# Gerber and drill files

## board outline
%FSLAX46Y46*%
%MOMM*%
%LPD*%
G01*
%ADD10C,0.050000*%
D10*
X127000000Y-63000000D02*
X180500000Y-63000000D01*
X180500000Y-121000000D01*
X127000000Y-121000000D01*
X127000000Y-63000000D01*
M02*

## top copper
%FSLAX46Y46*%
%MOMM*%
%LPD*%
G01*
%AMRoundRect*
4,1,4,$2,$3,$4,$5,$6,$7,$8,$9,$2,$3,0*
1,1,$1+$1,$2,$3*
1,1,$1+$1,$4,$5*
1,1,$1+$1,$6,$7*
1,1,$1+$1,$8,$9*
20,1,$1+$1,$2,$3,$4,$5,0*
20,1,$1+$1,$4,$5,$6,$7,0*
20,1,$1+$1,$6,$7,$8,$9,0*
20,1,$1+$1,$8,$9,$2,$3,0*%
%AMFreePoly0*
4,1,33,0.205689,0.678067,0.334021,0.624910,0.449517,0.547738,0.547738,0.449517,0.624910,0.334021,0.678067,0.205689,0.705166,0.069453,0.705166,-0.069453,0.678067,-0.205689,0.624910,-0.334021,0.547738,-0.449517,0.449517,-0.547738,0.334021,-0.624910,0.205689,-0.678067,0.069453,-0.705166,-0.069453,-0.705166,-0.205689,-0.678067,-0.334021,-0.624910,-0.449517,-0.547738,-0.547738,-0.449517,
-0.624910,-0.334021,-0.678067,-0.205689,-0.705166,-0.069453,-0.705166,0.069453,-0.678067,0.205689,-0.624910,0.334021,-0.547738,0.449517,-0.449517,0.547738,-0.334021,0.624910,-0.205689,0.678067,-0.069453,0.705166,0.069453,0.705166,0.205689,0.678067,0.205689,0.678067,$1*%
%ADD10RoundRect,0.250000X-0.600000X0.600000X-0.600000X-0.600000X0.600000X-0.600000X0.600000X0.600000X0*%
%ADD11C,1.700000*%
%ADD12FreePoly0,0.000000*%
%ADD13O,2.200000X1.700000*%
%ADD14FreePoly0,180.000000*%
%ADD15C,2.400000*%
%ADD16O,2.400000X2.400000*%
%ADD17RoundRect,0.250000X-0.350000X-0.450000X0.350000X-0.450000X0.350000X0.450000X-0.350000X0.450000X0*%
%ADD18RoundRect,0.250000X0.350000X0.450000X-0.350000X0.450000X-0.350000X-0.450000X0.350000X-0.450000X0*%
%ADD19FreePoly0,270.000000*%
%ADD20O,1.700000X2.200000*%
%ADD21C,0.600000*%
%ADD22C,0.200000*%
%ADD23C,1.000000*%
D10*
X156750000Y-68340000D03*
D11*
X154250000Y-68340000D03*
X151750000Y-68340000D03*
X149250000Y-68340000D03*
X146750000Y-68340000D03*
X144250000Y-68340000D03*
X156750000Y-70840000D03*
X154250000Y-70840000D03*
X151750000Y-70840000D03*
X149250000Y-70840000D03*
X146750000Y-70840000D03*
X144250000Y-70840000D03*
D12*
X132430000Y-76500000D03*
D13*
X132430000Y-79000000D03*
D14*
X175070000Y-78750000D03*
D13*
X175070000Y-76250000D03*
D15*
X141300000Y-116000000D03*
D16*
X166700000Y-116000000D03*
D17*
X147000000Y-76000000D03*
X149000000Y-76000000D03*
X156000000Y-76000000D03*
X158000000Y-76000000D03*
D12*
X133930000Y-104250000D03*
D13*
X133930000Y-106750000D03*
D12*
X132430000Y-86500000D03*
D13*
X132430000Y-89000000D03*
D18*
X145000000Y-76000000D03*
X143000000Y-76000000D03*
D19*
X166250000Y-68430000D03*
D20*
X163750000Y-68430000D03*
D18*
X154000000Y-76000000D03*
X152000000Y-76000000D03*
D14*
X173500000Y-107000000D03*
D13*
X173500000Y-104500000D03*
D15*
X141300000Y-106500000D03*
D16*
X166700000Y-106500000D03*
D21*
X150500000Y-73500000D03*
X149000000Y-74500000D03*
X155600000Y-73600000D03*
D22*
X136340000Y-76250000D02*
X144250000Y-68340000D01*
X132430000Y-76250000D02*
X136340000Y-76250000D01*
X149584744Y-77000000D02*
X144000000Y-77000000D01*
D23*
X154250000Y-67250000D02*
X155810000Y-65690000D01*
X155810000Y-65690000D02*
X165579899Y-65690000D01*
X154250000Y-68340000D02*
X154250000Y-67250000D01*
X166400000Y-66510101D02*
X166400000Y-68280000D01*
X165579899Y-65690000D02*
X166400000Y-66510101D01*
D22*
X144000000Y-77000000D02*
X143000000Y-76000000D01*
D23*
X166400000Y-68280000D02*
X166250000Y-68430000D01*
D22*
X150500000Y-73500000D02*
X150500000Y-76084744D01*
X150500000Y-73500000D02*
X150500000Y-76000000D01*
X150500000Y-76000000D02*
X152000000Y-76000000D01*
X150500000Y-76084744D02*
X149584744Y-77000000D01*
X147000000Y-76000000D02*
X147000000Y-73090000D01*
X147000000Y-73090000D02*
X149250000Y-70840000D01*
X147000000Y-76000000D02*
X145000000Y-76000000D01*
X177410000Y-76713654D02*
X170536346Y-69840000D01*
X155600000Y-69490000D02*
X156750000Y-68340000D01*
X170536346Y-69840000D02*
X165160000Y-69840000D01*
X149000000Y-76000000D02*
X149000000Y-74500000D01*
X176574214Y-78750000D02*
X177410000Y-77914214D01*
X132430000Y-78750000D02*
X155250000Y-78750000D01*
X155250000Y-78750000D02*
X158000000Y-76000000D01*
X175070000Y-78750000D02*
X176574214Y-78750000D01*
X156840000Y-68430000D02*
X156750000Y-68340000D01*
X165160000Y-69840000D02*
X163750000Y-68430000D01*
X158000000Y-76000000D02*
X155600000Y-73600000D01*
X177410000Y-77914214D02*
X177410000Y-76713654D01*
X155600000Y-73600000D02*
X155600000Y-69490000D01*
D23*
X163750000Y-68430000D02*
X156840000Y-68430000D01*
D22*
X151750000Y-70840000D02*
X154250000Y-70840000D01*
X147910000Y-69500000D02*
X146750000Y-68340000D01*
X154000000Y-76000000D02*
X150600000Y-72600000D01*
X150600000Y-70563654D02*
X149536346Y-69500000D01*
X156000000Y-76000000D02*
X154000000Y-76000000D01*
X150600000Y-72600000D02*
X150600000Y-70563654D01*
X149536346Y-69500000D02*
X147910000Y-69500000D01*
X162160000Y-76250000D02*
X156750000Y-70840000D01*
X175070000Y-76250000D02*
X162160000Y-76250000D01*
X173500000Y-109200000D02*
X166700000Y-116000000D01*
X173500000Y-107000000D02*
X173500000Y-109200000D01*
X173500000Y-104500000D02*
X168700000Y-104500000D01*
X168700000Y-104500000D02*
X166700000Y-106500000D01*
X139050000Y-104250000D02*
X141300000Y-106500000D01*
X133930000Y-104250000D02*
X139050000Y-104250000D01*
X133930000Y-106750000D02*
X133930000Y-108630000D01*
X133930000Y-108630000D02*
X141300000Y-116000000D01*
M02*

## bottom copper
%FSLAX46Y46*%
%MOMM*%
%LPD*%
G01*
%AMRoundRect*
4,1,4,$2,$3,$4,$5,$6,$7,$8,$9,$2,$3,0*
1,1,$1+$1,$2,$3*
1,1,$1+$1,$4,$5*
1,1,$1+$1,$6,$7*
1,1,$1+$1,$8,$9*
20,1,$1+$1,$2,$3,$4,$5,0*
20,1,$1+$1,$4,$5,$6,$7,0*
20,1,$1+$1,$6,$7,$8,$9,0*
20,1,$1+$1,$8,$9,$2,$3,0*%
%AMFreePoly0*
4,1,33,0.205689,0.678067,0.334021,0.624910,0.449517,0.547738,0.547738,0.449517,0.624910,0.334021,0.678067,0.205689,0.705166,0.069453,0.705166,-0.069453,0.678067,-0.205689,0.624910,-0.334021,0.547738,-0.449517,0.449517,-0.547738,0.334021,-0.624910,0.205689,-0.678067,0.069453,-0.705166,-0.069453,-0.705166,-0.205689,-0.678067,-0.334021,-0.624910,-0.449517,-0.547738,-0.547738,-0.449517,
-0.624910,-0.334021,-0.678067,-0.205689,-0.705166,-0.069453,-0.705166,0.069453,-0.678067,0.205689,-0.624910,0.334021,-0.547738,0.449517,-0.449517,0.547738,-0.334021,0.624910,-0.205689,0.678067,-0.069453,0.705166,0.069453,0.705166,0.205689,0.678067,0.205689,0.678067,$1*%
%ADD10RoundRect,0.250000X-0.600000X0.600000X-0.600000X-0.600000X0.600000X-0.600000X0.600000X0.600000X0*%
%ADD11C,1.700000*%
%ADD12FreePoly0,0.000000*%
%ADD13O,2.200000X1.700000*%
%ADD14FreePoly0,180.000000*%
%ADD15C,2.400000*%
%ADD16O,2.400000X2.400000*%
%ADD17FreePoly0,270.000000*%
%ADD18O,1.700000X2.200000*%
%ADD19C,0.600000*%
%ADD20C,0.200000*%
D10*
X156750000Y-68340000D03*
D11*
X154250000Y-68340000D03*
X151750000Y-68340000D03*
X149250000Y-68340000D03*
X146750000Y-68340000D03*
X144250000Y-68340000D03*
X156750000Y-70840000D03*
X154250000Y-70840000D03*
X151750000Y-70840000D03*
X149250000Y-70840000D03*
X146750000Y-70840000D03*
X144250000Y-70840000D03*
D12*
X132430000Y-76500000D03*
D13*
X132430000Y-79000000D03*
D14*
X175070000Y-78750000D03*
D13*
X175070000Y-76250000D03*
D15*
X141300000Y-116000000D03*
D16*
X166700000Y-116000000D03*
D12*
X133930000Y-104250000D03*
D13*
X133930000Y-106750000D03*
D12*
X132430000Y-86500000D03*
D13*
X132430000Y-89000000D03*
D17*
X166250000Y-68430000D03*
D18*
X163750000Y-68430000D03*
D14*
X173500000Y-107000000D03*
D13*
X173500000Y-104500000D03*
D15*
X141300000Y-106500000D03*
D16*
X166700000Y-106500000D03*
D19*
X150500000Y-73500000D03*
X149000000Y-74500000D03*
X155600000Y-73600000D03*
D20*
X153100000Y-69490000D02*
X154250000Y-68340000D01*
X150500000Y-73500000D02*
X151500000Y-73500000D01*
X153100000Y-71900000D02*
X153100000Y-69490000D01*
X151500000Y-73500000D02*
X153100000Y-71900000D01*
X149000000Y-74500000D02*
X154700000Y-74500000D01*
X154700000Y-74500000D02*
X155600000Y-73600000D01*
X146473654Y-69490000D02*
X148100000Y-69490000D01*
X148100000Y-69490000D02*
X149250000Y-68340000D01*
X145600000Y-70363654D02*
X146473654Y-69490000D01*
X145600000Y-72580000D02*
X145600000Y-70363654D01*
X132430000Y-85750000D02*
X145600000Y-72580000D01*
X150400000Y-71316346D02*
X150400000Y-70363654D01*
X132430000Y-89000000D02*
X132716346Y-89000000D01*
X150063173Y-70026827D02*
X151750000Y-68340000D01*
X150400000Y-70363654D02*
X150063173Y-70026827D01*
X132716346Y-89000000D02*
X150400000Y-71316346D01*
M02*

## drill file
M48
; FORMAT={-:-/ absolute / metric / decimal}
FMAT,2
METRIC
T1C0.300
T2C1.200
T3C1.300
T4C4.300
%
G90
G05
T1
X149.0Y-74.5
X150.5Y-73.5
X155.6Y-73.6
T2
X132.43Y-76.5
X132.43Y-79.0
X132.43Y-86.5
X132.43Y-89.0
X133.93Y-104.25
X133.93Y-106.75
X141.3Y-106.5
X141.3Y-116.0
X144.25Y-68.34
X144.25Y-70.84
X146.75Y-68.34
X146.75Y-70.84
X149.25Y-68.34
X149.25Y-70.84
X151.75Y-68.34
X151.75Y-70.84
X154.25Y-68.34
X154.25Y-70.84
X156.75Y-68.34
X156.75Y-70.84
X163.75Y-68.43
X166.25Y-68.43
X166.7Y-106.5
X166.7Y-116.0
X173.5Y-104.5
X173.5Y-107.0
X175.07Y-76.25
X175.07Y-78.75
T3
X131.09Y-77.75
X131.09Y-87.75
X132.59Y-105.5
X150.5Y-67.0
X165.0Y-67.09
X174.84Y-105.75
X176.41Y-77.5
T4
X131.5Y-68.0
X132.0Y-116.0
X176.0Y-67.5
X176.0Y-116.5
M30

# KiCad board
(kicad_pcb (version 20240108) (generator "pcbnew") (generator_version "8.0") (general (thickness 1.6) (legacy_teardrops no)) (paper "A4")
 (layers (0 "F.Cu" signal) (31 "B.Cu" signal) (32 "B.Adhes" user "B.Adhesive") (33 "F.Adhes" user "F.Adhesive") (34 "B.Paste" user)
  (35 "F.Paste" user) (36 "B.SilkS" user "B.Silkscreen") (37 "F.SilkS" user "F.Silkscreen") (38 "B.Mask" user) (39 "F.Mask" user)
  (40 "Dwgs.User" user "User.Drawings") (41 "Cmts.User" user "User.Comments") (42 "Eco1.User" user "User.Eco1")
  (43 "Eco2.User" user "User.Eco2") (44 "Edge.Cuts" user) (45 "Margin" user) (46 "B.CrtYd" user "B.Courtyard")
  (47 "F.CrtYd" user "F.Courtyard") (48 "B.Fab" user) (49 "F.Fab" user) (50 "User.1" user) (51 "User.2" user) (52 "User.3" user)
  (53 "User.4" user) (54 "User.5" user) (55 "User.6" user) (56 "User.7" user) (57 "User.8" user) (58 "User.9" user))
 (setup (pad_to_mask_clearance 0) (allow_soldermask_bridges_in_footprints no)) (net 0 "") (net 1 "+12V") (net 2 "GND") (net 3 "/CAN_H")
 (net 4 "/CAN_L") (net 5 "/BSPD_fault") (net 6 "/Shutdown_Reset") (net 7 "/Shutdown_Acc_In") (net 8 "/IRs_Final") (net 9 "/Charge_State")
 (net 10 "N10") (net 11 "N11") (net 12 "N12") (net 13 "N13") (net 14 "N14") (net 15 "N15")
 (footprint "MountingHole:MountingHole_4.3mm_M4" (layer "F.Cu") (at 176 116.5)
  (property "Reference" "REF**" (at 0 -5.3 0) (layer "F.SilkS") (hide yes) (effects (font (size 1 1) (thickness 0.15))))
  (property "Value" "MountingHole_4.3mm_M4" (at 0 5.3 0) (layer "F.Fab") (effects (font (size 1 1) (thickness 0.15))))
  (pad "" np_thru_hole circle (at 0 0) (size 4.3 4.3) (drill 4.3) (layers "*.Cu" "*.Mask")))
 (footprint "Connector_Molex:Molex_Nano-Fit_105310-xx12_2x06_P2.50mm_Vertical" (layer "F.Cu") (at 156.75 68.34 -90)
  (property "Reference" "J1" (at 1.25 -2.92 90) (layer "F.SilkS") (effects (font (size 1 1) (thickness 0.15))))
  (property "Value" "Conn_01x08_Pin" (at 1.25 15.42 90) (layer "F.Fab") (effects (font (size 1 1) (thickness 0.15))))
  (pad "" np_thru_hole circle (at -1.34 6.25 270) (size 1.3 1.3) (drill 1.3) (layers "*.Cu" "*.Mask"))
  (pad "1" thru_hole roundrect (at 0 0 270) (size 1.7 1.7) (drill 1.2) (layers "*.Cu" "*.Mask") (remove_unused_layers no)
   (roundrect_rratio 0.147059) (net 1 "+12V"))
  (pad "2" thru_hole circle (at 0 2.5 270) (size 1.7 1.7) (drill 1.2) (layers "*.Cu" "*.Mask") (remove_unused_layers no) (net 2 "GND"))
  (pad "3" thru_hole circle (at 0 5 270) (size 1.7 1.7) (drill 1.2) (layers "*.Cu" "*.Mask") (remove_unused_layers no) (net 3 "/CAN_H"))
  (pad "4" thru_hole circle (at 0 7.5 270) (size 1.7 1.7) (drill 1.2) (layers "*.Cu" "*.Mask") (remove_unused_layers no) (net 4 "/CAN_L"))
  (pad "5" thru_hole circle (at 0 10 270) (size 1.7 1.7) (drill 1.2) (layers "*.Cu" "*.Mask") (remove_unused_layers no)
   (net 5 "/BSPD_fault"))
  (pad "6" thru_hole circle (at 0 12.5 270) (size 1.7 1.7) (drill 1.2) (layers "*.Cu" "*.Mask") (remove_unused_layers no)
   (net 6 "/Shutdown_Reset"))
  (pad "7" thru_hole circle (at 2.5 0 270) (size 1.7 1.7) (drill 1.2) (layers "*.Cu" "*.Mask") (remove_unused_layers no)
   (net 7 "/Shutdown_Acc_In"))
  (pad "8" thru_hole circle (at 2.5 2.5 270) (size 1.7 1.7) (drill 1.2) (layers "*.Cu" "*.Mask") (remove_unused_layers no)
   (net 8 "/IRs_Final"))
  (pad "9" thru_hole circle (at 2.5 5 270) (size 1.7 1.7) (drill 1.2) (layers "*.Cu" "*.Mask") (remove_unused_layers no)
   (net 8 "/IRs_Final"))
  (pad "10" thru_hole circle (at 2.5 7.5 270) (size 1.7 1.7) (drill 1.2) (layers "*.Cu" "*.Mask") (remove_unused_layers no)
   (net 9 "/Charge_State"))
  (pad "11" thru_hole circle (at 2.5 10 270) (size 1.7 1.7) (drill 1.2) (layers "*.Cu" "*.Mask") (remove_unused_layers no) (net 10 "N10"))
  (pad "12" thru_hole circle (at 2.5 12.5 270) (size 1.7 1.7) (drill 1.2) (layers "*.Cu" "*.Mask") (remove_unused_layers no) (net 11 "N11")))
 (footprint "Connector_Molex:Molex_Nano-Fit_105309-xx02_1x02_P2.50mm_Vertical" (layer "F.Cu") (at 132.43 76.5)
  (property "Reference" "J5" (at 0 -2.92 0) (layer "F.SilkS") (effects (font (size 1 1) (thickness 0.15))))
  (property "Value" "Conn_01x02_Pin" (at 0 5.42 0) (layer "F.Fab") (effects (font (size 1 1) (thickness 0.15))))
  (pad "" np_thru_hole circle (at -1.34 1.25) (size 1.3 1.3) (drill 1.3) (layers "*.Cu" "*.Mask"))
  (pad "1" thru_hole custom (at 0 0) (size 1.417157 1.417157) (drill 1.2) (layers "*.Cu" "*.Mask") (remove_unused_layers no)
   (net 6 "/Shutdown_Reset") (thermal_bridge_angle 90) (options (clearance outline) (anchor circle)) (primitives))
  (pad "2" thru_hole oval (at 0 2.5) (size 2.2 1.7) (drill 1.2) (layers "*.Cu" "*.Mask") (remove_unused_layers no) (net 1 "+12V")))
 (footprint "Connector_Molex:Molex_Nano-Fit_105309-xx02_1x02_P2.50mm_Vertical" (layer "F.Cu") (at 175.07 78.75 180)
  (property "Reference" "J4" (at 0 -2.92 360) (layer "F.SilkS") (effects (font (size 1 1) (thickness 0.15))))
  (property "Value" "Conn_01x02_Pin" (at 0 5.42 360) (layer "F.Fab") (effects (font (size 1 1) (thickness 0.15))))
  (pad "" np_thru_hole circle (at -1.34 1.25 180) (size 1.3 1.3) (drill 1.3) (layers "*.Cu" "*.Mask"))
  (pad "1" thru_hole custom (at 0 0 180) (size 1.417157 1.417157) (drill 1.2) (layers "*.Cu" "*.Mask") (remove_unused_layers no)
   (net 1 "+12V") (thermal_bridge_angle 90) (options (clearance outline) (anchor circle)) (primitives))
  (pad "2" thru_hole oval (at 0 2.5 180) (size 2.2 1.7) (drill 1.2) (layers "*.Cu" "*.Mask") (remove_unused_layers no)
   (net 7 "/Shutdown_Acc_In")))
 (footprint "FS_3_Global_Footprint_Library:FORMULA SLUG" (layer "F.Cu") (at 146 87.975292)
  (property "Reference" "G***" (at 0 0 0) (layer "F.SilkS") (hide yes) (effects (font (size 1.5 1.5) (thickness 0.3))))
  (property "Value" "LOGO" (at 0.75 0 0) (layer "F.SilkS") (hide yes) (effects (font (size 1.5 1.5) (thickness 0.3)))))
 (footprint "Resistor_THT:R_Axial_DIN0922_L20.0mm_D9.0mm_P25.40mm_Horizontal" (layer "F.Cu") (at 141.3 116)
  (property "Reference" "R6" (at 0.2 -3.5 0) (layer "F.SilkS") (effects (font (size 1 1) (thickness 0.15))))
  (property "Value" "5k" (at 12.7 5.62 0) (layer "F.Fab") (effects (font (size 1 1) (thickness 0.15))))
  (pad "1" thru_hole circle (at 0 0) (size 2.4 2.4) (drill 1.2) (layers "*.Cu" "*.Mask") (remove_unused_layers no) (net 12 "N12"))
  (pad "2" thru_hole oval (at 25.4 0) (size 2.4 2.4) (drill 1.2) (layers "*.Cu" "*.Mask") (remove_unused_layers no) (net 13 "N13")))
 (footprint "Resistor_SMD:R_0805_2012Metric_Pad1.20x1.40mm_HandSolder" (layer "F.Cu") (at 148 76)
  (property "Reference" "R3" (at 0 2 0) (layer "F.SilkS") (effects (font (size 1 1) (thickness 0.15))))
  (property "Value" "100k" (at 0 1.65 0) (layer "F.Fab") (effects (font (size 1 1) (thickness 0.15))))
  (pad "1" smd roundrect (at -1 0) (size 1.2 1.4) (layers "F.Cu" "F.Paste" "F.Mask") (roundrect_rratio 0.208333) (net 9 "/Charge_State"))
  (pad "2" smd roundrect (at 1 0) (size 1.2 1.4) (layers "F.Cu" "F.Paste" "F.Mask") (roundrect_rratio 0.208333) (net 1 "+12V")))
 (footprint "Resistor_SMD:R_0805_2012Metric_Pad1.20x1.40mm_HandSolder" (layer "F.Cu") (at 157 76)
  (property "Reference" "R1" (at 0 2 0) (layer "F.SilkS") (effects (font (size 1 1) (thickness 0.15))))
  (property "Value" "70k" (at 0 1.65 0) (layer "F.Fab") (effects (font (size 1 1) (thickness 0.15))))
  (pad "1" smd roundrect (at -1 0) (size 1.2 1.4) (layers "F.Cu" "F.Paste" "F.Mask") (roundrect_rratio 0.208333) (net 5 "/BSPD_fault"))
  (pad "2" smd roundrect (at 1 0) (size 1.2 1.4) (layers "F.Cu" "F.Paste" "F.Mask") (roundrect_rratio 0.208333) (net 1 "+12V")))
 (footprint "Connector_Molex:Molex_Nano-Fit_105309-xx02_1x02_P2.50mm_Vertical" (layer "F.Cu") (at 133.93 104.25)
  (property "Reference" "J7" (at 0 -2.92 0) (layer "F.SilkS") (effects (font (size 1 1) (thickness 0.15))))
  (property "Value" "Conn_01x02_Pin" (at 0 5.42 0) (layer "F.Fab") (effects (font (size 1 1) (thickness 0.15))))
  (pad "" np_thru_hole circle (at -1.34 1.25) (size 1.3 1.3) (drill 1.3) (layers "*.Cu" "*.Mask"))
  (pad "1" thru_hole custom (at 0 0) (size 1.417157 1.417157) (drill 1.2) (layers "*.Cu" "*.Mask") (remove_unused_layers no) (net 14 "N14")
   (thermal_bridge_angle 90) (options (clearance outline) (anchor circle)) (primitives))
  (pad "2" thru_hole oval (at 0 2.5) (size 2.2 1.7) (drill 1.2) (layers "*.Cu" "*.Mask") (remove_unused_layers no) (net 12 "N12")))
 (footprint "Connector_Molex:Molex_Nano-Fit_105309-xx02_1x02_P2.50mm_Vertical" (layer "F.Cu") (at 132.43 86.5)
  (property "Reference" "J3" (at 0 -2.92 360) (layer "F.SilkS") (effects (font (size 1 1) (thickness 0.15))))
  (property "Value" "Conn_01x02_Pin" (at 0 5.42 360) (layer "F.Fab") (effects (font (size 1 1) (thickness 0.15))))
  (pad "" np_thru_hole circle (at -1.34 1.25) (size 1.3 1.3) (drill 1.3) (layers "*.Cu" "*.Mask"))
  (pad "1" thru_hole custom (at 0 0) (size 1.417157 1.417157) (drill 1.2) (layers "*.Cu" "*.Mask") (remove_unused_layers no)
   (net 4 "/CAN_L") (thermal_bridge_angle 90) (options (clearance outline) (anchor circle)) (primitives))
  (pad "2" thru_hole oval (at 0 2.5) (size 2.2 1.7) (drill 1.2) (layers "*.Cu" "*.Mask") (remove_unused_layers no) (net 3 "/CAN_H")))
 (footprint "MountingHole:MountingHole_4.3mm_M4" (layer "F.Cu") (at 132 116)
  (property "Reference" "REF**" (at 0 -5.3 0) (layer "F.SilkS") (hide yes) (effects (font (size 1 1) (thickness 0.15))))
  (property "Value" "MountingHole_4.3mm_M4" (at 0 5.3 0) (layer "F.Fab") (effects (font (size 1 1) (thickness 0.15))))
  (pad "" np_thru_hole circle (at 0 0) (size 4.3 4.3) (drill 4.3) (layers "*.Cu" "*.Mask")))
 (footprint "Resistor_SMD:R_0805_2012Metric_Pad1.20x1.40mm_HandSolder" (layer "F.Cu") (at 144 76 180)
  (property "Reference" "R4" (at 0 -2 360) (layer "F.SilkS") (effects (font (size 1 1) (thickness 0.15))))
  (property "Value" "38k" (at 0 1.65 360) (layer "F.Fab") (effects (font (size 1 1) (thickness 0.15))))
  (pad "1" smd roundrect (at -1 0 180) (size 1.2 1.4) (layers "F.Cu" "F.Paste" "F.Mask") (roundrect_rratio 0.208333) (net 9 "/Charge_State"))
  (pad "2" smd roundrect (at 1 0 180) (size 1.2 1.4) (layers "F.Cu" "F.Paste" "F.Mask") (roundrect_rratio 0.208333) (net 2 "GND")))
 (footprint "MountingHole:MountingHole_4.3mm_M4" (layer "F.Cu") (at 131.5 68)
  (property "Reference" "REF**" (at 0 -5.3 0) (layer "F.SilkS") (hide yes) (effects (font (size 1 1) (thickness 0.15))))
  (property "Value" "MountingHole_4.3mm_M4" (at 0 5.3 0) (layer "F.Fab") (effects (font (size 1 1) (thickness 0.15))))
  (pad "" np_thru_hole circle (at 0 0) (size 4.3 4.3) (drill 4.3) (layers "*.Cu" "*.Mask")))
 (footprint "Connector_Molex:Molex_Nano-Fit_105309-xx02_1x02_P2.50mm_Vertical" (layer "F.Cu") (at 166.25 68.43 -90)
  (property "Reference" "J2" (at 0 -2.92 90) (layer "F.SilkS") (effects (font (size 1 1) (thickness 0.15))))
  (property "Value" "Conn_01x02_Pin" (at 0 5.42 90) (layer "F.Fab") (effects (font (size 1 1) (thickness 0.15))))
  (pad "" np_thru_hole circle (at -1.34 1.25 270) (size 1.3 1.3) (drill 1.3) (layers "*.Cu" "*.Mask"))
  (pad "1" thru_hole custom (at 0 0 270) (size 1.417157 1.417157) (drill 1.2) (layers "*.Cu" "*.Mask") (remove_unused_layers no)
   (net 2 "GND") (thermal_bridge_angle 90) (options (clearance outline) (anchor circle)) (primitives))
  (pad "2" thru_hole oval (at 0 2.5 270) (size 2.2 1.7) (drill 1.2) (layers "*.Cu" "*.Mask") (remove_unused_layers no) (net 1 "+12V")))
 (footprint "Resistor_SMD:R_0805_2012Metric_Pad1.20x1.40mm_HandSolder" (layer "F.Cu") (at 153 76 180)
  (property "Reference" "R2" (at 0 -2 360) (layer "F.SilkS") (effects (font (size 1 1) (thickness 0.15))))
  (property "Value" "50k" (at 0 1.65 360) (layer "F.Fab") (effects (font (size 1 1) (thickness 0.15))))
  (pad "1" smd roundrect (at -1 0 180) (size 1.2 1.4) (layers "F.Cu" "F.Paste" "F.Mask") (roundrect_rratio 0.208333) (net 5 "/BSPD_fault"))
  (pad "2" smd roundrect (at 1 0 180) (size 1.2 1.4) (layers "F.Cu" "F.Paste" "F.Mask") (roundrect_rratio 0.208333) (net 2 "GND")))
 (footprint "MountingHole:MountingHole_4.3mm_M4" (layer "F.Cu") (at 176 67.5)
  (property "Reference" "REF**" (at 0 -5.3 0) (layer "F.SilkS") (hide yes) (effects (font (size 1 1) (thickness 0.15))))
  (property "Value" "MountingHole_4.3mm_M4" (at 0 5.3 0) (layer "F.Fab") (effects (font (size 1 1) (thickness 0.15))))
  (pad "" np_thru_hole circle (at 0 0) (size 4.3 4.3) (drill 4.3) (layers "*.Cu" "*.Mask")))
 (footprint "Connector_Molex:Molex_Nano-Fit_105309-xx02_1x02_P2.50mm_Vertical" (layer "F.Cu") (at 173.5 107 180)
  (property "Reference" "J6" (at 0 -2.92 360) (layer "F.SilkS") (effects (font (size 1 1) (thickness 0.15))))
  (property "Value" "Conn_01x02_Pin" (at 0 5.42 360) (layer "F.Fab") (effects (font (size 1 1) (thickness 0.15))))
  (pad "" np_thru_hole circle (at -1.34 1.25 180) (size 1.3 1.3) (drill 1.3) (layers "*.Cu" "*.Mask"))
  (pad "1" thru_hole custom (at 0 0 180) (size 1.417157 1.417157) (drill 1.2) (layers "*.Cu" "*.Mask") (remove_unused_layers no)
   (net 13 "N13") (thermal_bridge_angle 90) (options (clearance outline) (anchor circle)) (primitives))
  (pad "2" thru_hole oval (at 0 2.5 180) (size 2.2 1.7) (drill 1.2) (layers "*.Cu" "*.Mask") (remove_unused_layers no) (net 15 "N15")))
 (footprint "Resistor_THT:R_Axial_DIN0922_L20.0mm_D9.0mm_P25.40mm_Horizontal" (layer "F.Cu") (at 141.3 106.5)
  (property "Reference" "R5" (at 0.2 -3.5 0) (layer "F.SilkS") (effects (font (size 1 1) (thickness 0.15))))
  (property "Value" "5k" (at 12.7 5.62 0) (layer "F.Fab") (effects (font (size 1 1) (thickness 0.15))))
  (pad "1" thru_hole circle (at 0 0) (size 2.4 2.4) (drill 1.2) (layers "*.Cu" "*.Mask") (remove_unused_layers no) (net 14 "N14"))
  (pad "2" thru_hole oval (at 25.4 0) (size 2.4 2.4) (drill 1.2) (layers "*.Cu" "*.Mask") (remove_unused_layers no) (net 15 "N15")))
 (gr_rect (start 127 63) (end 180.5 121) (stroke (width 0.05) (type default)) (fill none) (layer "Edge.Cuts"))
 (segment (start 136.34 76.25) (end 144.25 68.34) (width 0.2) (layer "F.Cu") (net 6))
 (segment (start 132.43 76.25) (end 136.34 76.25) (width 0.2) (layer "F.Cu") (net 6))
 (segment (start 149.584744 77) (end 144 77) (width 0.2) (layer "F.Cu") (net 2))
 (segment (start 154.25 67.25) (end 155.81 65.69) (width 1) (layer "F.Cu") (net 2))
 (segment (start 155.81 65.69) (end 165.579899 65.69) (width 1) (layer "F.Cu") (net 2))
 (segment (start 154.25 68.34) (end 154.25 67.25) (width 1) (layer "F.Cu") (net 2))
 (segment (start 166.4 66.510101) (end 166.4 68.28) (width 1) (layer "F.Cu") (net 2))
 (segment (start 165.579899 65.69) (end 166.4 66.510101) (width 1) (layer "F.Cu") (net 2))
 (segment (start 144 77) (end 143 76) (width 0.2) (layer "F.Cu") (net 2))
 (segment (start 166.4 68.28) (end 166.25 68.43) (width 1) (layer "F.Cu") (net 2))
 (segment (start 150.5 73.5) (end 150.5 76.084744) (width 0.2) (layer "F.Cu") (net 2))
 (segment (start 150.5 73.5) (end 150.5 76) (width 0.2) (layer "F.Cu") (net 2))
 (segment (start 150.5 76) (end 152 76) (width 0.2) (layer "F.Cu") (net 2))
 (segment (start 150.5 76.084744) (end 149.584744 77) (width 0.2) (layer "F.Cu") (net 2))
 (via (at 150.5 73.5) (size 0.6) (drill 0.3) (layers "F.Cu" "B.Cu") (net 2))
 (segment (start 153.1 69.49) (end 154.25 68.34) (width 0.2) (layer "B.Cu") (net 2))
 (segment (start 150.5 73.5) (end 151.5 73.5) (width 0.2) (layer "B.Cu") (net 2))
 (segment (start 153.1 71.9) (end 153.1 69.49) (width 0.2) (layer "B.Cu") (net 2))
 (segment (start 151.5 73.5) (end 153.1 71.9) (width 0.2) (layer "B.Cu") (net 2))
 (segment (start 147 76) (end 147 73.09) (width 0.2) (layer "F.Cu") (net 9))
 (segment (start 147 73.09) (end 149.25 70.84) (width 0.2) (layer "F.Cu") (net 9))
 (segment (start 147 76) (end 145 76) (width 0.2) (layer "F.Cu") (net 9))
 (segment (start 177.41 76.713654) (end 170.536346 69.84) (width 0.2) (layer "F.Cu") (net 1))
 (segment (start 155.6 69.49) (end 156.75 68.34) (width 0.2) (layer "F.Cu") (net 1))
 (segment (start 170.536346 69.84) (end 165.16 69.84) (width 0.2) (layer "F.Cu") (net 1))
 (segment (start 149 76) (end 149 74.5) (width 0.2) (layer "F.Cu") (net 1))
 (segment (start 176.574214 78.75) (end 177.41 77.914214) (width 0.2) (layer "F.Cu") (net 1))
 (segment (start 132.43 78.75) (end 155.25 78.75) (width 0.2) (layer "F.Cu") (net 1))
 (segment (start 155.25 78.75) (end 158 76) (width 0.2) (layer "F.Cu") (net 1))
 (segment (start 175.07 78.75) (end 176.574214 78.75) (width 0.2) (layer "F.Cu") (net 1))
 (segment (start 156.84 68.43) (end 156.75 68.34) (width 0.2) (layer "F.Cu") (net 1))
 (segment (start 165.16 69.84) (end 163.75 68.43) (width 0.2) (layer "F.Cu") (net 1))
 (segment (start 158 76) (end 155.6 73.6) (width 0.2) (layer "F.Cu") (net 1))
 (segment (start 177.41 77.914214) (end 177.41 76.713654) (width 0.2) (layer "F.Cu") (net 1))
 (segment (start 155.6 73.6) (end 155.6 69.49) (width 0.2) (layer "F.Cu") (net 1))
 (segment (start 163.75 68.43) (end 156.84 68.43) (width 1) (layer "F.Cu") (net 1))
 (via (at 149 74.5) (size 0.6) (drill 0.3) (layers "F.Cu" "B.Cu") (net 1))
 (via (at 155.6 73.6) (size 0.6) (drill 0.3) (layers "F.Cu" "B.Cu") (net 1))
 (segment (start 149 74.5) (end 154.7 74.5) (width 0.2) (layer "B.Cu") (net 1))
 (segment (start 154.7 74.5) (end 155.6 73.6) (width 0.2) (layer "B.Cu") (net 1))
 (segment (start 151.75 70.84) (end 154.25 70.84) (width 0.2) (layer "F.Cu") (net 8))
 (segment (start 147.91 69.5) (end 146.75 68.34) (width 0.2) (layer "F.Cu") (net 5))
 (segment (start 154 76) (end 150.6 72.6) (width 0.2) (layer "F.Cu") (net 5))
 (segment (start 150.6 70.563654) (end 149.536346 69.5) (width 0.2) (layer "F.Cu") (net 5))
 (segment (start 156 76) (end 154 76) (width 0.2) (layer "F.Cu") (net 5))
 (segment (start 150.6 72.6) (end 150.6 70.563654) (width 0.2) (layer "F.Cu") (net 5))
 (segment (start 149.536346 69.5) (end 147.91 69.5) (width 0.2) (layer "F.Cu") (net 5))
 (segment (start 146.473654 69.49) (end 148.1 69.49) (width 0.2) (layer "B.Cu") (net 4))
 (segment (start 148.1 69.49) (end 149.25 68.34) (width 0.2) (layer "B.Cu") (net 4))
 (segment (start 145.6 70.363654) (end 146.473654 69.49) (width 0.2) (layer "B.Cu") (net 4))
 (segment (start 145.6 72.58) (end 145.6 70.363654) (width 0.2) (layer "B.Cu") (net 4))
 (segment (start 132.43 85.75) (end 145.6 72.58) (width 0.2) (layer "B.Cu") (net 4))
 (segment (start 162.16 76.25) (end 156.75 70.84) (width 0.2) (layer "F.Cu") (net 7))
 (segment (start 175.07 76.25) (end 162.16 76.25) (width 0.2) (layer "F.Cu") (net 7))
 (segment (start 150.4 71.316346) (end 150.4 70.363654) (width 0.2) (layer "B.Cu") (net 3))
 (segment (start 132.43 89) (end 132.716346 89) (width 0.2) (layer "B.Cu") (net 3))
 (segment (start 150.063173 70.026827) (end 151.75 68.34) (width 0.2) (layer "B.Cu") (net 3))
 (segment (start 150.4 70.363654) (end 150.063173 70.026827) (width 0.2) (layer "B.Cu") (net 3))
 (segment (start 132.716346 89) (end 150.4 71.316346) (width 0.2) (layer "B.Cu") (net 3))
 (segment (start 173.5 109.2) (end 166.7 116) (width 0.2) (layer "F.Cu") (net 13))
 (segment (start 173.5 107) (end 173.5 109.2) (width 0.2) (layer "F.Cu") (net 13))
 (segment (start 173.5 104.5) (end 168.7 104.5) (width 0.2) (layer "F.Cu") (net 15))
 (segment (start 168.7 104.5) (end 166.7 106.5) (width 0.2) (layer "F.Cu") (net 15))
 (segment (start 139.05 104.25) (end 141.3 106.5) (width 0.2) (layer "F.Cu") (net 14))
 (segment (start 133.93 104.25) (end 139.05 104.25) (width 0.2) (layer "F.Cu") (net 14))
 (segment (start 133.93 106.75) (end 133.93 108.63) (width 0.2) (layer "F.Cu") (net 12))
 (segment (start 133.93 108.63) (end 141.3 116) (width 0.2) (layer "F.Cu") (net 12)))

